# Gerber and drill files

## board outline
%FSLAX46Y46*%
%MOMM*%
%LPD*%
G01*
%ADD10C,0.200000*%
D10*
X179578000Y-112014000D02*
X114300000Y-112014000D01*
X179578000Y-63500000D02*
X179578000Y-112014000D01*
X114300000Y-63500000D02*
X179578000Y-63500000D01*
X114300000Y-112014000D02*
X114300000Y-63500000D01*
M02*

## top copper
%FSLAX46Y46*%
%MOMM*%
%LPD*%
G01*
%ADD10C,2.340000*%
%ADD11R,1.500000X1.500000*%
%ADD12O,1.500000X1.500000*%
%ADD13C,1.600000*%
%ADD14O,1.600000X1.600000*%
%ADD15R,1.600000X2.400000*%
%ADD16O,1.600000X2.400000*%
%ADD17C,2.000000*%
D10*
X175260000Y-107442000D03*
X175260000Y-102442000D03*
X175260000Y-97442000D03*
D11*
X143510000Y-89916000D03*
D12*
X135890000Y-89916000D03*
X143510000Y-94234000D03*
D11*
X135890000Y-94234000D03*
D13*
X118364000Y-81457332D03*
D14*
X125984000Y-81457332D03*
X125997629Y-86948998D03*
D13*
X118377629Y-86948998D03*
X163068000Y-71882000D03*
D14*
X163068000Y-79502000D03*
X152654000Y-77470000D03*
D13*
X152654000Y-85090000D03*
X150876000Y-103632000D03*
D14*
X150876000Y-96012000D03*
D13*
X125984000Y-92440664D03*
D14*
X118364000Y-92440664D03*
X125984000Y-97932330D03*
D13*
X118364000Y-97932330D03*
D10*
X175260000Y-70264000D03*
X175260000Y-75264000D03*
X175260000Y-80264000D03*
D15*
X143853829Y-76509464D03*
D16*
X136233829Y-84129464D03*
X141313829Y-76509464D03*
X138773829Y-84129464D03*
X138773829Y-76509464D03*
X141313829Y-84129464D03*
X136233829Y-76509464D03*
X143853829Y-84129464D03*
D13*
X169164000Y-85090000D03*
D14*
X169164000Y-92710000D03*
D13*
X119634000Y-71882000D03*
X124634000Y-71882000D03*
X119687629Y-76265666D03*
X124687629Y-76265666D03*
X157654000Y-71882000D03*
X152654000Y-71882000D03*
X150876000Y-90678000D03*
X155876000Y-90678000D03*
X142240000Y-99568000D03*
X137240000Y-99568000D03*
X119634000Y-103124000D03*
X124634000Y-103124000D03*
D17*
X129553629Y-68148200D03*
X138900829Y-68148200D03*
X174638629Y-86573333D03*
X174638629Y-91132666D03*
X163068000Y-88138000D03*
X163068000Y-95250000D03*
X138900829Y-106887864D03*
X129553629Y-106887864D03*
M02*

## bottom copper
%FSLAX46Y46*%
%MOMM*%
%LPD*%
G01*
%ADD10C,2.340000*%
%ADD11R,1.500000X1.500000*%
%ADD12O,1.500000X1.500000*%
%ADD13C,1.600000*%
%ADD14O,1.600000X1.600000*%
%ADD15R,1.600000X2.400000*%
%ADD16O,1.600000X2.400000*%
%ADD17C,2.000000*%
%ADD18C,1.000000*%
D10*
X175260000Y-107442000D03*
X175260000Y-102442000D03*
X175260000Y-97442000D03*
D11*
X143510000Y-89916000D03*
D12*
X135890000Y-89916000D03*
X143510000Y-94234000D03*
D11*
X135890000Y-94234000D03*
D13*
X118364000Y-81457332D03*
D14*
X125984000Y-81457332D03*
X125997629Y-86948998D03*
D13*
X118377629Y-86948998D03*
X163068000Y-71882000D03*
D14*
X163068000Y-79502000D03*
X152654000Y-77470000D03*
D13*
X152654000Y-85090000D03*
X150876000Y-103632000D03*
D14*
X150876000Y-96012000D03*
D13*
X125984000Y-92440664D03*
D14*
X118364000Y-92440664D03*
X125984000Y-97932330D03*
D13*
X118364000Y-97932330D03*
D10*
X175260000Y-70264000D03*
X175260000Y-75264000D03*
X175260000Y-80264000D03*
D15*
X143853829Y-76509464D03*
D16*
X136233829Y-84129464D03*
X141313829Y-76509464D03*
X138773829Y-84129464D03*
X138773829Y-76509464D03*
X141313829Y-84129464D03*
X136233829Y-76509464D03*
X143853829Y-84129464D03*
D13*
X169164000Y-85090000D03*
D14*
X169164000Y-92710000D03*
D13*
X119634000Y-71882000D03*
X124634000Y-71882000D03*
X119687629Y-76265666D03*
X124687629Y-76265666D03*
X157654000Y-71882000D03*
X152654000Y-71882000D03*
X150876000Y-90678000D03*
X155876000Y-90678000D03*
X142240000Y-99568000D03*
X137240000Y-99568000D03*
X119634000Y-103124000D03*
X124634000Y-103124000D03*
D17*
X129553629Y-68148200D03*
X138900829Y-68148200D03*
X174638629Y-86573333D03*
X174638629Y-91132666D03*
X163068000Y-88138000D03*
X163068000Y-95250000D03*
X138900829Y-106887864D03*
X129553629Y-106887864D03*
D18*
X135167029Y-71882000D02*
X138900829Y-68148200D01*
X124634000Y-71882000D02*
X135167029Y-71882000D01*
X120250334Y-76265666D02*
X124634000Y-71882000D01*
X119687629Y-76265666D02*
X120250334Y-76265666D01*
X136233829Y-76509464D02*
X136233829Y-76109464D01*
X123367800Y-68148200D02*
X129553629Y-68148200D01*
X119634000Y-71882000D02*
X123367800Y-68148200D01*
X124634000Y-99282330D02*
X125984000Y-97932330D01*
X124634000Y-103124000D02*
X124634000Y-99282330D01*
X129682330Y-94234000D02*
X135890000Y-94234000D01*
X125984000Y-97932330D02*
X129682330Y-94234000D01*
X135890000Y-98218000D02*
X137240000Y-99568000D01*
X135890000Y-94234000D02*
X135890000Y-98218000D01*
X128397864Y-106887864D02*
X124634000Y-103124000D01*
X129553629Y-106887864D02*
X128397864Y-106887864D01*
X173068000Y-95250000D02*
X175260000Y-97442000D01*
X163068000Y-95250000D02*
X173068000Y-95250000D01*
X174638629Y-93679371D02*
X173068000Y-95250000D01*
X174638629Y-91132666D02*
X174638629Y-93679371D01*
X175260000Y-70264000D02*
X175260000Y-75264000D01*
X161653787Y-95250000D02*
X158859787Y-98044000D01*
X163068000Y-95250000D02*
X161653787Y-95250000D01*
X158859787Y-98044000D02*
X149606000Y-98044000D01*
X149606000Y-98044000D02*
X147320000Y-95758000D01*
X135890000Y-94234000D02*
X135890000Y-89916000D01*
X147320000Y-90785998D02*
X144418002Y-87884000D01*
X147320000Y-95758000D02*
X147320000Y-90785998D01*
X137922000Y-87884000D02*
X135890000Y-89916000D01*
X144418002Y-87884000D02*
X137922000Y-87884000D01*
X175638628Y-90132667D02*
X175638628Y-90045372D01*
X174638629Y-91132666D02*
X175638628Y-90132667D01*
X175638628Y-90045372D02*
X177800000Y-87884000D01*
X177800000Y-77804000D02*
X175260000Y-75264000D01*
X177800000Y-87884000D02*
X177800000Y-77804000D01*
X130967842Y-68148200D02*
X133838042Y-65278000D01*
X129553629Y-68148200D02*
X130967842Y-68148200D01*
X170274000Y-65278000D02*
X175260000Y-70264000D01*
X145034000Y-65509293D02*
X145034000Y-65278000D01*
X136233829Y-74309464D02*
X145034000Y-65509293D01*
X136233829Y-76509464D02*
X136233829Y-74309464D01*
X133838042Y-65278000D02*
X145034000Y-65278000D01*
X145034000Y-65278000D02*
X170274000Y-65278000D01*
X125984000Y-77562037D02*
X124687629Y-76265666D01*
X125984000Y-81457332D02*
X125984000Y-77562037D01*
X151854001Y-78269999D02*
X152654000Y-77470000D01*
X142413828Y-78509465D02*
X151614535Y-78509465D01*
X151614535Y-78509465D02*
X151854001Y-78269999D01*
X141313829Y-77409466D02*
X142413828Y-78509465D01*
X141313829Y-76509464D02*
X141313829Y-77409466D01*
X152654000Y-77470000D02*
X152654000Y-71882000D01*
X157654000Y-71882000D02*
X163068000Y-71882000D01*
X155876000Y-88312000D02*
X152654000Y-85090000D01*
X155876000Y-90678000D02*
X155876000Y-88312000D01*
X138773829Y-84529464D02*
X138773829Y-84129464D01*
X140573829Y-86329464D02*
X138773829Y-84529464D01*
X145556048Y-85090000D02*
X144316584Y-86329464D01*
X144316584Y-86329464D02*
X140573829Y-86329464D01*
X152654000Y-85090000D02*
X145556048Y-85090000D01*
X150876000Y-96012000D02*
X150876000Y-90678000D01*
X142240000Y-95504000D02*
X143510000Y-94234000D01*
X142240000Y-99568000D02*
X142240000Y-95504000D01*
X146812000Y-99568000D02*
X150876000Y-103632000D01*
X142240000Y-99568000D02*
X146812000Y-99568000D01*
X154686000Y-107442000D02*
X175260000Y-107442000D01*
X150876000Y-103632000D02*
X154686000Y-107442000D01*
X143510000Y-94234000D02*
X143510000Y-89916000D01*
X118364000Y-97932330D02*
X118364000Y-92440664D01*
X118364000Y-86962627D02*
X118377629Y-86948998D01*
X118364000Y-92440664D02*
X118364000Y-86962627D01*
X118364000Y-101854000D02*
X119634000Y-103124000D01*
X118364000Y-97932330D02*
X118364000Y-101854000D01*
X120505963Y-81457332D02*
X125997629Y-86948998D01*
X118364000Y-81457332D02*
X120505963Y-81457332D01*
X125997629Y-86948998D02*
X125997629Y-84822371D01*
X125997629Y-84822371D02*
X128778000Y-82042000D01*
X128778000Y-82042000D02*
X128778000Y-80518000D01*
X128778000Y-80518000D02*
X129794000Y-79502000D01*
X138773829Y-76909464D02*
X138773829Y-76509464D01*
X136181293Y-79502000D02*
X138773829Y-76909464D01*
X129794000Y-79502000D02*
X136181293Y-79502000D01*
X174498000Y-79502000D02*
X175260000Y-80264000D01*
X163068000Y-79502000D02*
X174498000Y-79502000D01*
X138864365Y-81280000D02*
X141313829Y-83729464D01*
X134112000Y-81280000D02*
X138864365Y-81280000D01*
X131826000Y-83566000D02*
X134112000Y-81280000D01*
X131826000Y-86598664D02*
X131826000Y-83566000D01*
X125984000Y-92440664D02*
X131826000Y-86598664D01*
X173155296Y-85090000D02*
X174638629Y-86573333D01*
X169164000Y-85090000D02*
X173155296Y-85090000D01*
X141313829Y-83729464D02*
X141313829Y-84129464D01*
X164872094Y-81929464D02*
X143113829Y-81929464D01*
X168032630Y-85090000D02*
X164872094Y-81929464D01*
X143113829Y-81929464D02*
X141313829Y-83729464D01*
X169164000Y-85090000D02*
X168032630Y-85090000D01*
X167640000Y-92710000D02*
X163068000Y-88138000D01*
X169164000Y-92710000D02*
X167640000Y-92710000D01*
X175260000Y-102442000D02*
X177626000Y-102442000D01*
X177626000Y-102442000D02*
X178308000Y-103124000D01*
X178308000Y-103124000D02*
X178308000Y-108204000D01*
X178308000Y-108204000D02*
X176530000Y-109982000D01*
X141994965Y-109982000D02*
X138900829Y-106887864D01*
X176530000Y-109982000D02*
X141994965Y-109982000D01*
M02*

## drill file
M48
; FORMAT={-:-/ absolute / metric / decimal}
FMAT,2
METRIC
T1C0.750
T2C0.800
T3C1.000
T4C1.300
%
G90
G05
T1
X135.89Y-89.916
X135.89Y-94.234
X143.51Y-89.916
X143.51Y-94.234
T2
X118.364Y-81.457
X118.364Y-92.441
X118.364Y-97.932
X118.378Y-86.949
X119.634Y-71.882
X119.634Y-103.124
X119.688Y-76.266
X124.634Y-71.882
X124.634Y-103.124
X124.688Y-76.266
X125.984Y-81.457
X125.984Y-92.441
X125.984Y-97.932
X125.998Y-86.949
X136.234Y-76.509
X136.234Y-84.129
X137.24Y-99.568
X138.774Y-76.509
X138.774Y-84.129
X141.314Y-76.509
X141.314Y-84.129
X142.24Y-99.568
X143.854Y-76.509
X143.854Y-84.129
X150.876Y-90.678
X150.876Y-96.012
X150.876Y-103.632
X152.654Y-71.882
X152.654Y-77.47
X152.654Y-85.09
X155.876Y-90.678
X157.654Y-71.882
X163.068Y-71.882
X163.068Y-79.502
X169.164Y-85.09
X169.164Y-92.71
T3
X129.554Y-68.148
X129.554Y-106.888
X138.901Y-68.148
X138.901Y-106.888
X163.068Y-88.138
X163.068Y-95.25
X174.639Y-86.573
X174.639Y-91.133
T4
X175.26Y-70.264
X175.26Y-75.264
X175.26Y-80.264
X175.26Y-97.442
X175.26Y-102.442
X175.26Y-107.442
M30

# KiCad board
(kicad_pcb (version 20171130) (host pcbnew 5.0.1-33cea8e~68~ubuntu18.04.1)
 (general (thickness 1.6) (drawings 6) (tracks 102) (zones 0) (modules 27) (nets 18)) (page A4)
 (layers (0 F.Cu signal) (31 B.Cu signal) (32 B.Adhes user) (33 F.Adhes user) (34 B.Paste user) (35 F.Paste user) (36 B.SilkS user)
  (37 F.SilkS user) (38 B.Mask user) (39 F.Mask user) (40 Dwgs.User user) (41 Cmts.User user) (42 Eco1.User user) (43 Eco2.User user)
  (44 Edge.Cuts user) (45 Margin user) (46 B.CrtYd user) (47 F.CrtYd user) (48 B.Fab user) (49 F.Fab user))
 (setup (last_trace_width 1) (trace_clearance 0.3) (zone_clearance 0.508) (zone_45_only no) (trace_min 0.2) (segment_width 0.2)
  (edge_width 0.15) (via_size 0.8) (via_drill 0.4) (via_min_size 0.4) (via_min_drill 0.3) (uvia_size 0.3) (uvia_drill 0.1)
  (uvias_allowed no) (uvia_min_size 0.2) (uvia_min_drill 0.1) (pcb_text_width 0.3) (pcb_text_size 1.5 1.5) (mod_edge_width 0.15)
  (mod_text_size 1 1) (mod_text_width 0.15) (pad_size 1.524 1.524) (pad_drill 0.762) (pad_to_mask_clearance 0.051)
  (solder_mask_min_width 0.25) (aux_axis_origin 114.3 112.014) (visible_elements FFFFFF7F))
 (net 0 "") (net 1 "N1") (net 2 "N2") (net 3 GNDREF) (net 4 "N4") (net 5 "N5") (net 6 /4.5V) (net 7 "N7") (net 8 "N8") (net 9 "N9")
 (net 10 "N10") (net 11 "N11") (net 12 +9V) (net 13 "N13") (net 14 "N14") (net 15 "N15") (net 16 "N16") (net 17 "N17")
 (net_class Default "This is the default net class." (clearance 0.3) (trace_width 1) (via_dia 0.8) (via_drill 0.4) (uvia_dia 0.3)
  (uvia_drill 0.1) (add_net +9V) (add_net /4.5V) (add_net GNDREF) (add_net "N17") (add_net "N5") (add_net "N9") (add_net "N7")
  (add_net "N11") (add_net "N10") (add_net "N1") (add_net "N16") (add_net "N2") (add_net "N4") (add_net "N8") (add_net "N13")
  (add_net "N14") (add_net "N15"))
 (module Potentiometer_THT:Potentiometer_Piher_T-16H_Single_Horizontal (layer F.Cu) (at 175.26 107.442)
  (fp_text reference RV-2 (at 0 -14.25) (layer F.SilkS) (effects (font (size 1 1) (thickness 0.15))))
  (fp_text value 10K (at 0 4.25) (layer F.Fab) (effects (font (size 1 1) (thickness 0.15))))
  (pad 1 thru_hole circle (at 0 0) (size 2.34 2.34) (drill 1.3) (layers *.Cu *.Mask) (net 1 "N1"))
  (pad 2 thru_hole circle (at 0 -5) (size 2.34 2.34) (drill 1.3) (layers *.Cu *.Mask) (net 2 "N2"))
  (pad 3 thru_hole circle (at 0 -10) (size 2.34 2.34) (drill 1.3) (layers *.Cu *.Mask) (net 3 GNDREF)))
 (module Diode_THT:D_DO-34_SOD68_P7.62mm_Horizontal (layer F.Cu) (at 143.51 89.916 180)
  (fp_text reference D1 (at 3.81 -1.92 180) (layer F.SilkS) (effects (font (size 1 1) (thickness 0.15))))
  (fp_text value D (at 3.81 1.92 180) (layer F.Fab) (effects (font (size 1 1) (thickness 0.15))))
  (pad 1 thru_hole rect (at 0 0 180) (size 1.5 1.5) (drill 0.75) (layers *.Cu *.Mask) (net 1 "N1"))
  (pad 2 thru_hole oval (at 7.62 0 180) (size 1.5 1.5) (drill 0.75) (layers *.Cu *.Mask) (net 3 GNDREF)))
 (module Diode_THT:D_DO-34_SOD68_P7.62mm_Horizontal (layer F.Cu) (at 135.89 94.234)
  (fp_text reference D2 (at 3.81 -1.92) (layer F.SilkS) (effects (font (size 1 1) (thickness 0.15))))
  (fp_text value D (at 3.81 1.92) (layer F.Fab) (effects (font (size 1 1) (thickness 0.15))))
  (pad 2 thru_hole oval (at 7.62 0) (size 1.5 1.5) (drill 0.75) (layers *.Cu *.Mask) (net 1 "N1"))
  (pad 1 thru_hole rect (at 0 0) (size 1.5 1.5) (drill 0.75) (layers *.Cu *.Mask) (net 3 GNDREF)))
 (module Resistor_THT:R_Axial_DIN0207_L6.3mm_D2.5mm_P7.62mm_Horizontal (layer F.Cu) (at 118.364 81.457332)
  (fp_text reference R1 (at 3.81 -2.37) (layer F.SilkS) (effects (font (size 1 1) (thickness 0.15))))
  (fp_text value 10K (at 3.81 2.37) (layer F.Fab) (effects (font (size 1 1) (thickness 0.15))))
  (pad 1 thru_hole circle (at 0 0) (size 1.6 1.6) (drill 0.8) (layers *.Cu *.Mask) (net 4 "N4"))
  (pad 2 thru_hole oval (at 7.62 0) (size 1.6 1.6) (drill 0.8) (layers *.Cu *.Mask) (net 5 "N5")))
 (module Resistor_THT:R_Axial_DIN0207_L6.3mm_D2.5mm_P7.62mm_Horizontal (layer F.Cu) (at 118.377629 86.948998)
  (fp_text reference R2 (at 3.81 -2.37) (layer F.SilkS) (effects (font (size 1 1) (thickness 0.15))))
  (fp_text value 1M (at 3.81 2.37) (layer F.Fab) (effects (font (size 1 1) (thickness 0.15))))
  (pad 2 thru_hole oval (at 7.62 0) (size 1.6 1.6) (drill 0.8) (layers *.Cu *.Mask) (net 4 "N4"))
  (pad 1 thru_hole circle (at 0 0) (size 1.6 1.6) (drill 0.8) (layers *.Cu *.Mask) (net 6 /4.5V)))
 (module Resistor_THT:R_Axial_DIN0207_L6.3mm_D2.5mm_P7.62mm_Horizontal (layer F.Cu) (at 163.068 71.882 270)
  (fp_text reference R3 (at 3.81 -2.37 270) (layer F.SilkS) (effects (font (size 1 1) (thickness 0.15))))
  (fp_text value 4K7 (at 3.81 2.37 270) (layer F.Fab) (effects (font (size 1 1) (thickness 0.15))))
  (pad 1 thru_hole circle (at 0 0 270) (size 1.6 1.6) (drill 0.8) (layers *.Cu *.Mask) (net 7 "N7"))
  (pad 2 thru_hole oval (at 7.62 0 270) (size 1.6 1.6) (drill 0.8) (layers *.Cu *.Mask) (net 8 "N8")))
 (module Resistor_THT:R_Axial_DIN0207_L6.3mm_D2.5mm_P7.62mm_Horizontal (layer F.Cu) (at 152.654 85.09 90)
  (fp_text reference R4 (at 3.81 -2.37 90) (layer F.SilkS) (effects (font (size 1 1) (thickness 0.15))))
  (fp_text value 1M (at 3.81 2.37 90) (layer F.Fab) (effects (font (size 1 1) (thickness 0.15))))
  (pad 2 thru_hole oval (at 7.62 0 90) (size 1.6 1.6) (drill 0.8) (layers *.Cu *.Mask) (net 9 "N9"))
  (pad 1 thru_hole circle (at 0 0 90) (size 1.6 1.6) (drill 0.8) (layers *.Cu *.Mask) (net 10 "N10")))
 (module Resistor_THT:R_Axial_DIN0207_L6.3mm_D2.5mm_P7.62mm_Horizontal (layer F.Cu) (at 150.876 103.632 90)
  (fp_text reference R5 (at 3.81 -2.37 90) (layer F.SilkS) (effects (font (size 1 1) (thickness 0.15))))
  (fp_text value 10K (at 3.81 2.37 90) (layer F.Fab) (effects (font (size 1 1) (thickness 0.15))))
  (pad 1 thru_hole circle (at 0 0 90) (size 1.6 1.6) (drill 0.8) (layers *.Cu *.Mask) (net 1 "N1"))
  (pad 2 thru_hole oval (at 7.62 0 90) (size 1.6 1.6) (drill 0.8) (layers *.Cu *.Mask) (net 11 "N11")))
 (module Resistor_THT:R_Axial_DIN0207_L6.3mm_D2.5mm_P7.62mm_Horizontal (layer F.Cu) (at 125.984 92.440664 180)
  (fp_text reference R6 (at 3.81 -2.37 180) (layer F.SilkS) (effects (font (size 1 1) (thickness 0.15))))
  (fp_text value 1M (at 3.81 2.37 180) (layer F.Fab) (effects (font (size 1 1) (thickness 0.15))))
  (pad 1 thru_hole circle (at 0 0 180) (size 1.6 1.6) (drill 0.8) (layers *.Cu *.Mask) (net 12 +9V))
  (pad 2 thru_hole oval (at 7.62 0 180) (size 1.6 1.6) (drill 0.8) (layers *.Cu *.Mask) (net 6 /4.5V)))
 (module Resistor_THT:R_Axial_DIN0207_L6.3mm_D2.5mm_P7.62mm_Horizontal (layer F.Cu) (at 118.364 97.93233)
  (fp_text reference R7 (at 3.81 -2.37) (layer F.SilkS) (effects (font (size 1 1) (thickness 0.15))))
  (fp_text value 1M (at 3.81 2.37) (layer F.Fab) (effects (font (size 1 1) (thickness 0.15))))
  (pad 2 thru_hole oval (at 7.62 0) (size 1.6 1.6) (drill 0.8) (layers *.Cu *.Mask) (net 3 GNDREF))
  (pad 1 thru_hole circle (at 0 0) (size 1.6 1.6) (drill 0.8) (layers *.Cu *.Mask) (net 6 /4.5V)))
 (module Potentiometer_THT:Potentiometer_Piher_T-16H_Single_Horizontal (layer F.Cu) (at 175.26 80.264)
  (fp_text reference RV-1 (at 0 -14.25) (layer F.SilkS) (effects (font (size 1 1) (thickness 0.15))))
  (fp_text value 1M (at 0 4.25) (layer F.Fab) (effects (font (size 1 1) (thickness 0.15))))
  (pad 3 thru_hole circle (at 0 -10) (size 2.34 2.34) (drill 1.3) (layers *.Cu *.Mask) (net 3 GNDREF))
  (pad 2 thru_hole circle (at 0 -5) (size 2.34 2.34) (drill 1.3) (layers *.Cu *.Mask) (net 3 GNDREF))
  (pad 1 thru_hole circle (at 0 0) (size 2.34 2.34) (drill 1.3) (layers *.Cu *.Mask) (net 8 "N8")))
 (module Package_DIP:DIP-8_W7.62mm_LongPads (layer F.Cu) (at 143.853829 76.509464 270)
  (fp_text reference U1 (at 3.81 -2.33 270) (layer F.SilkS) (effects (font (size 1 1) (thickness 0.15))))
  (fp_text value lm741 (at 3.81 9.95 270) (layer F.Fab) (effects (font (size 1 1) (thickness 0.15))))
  (pad 1 thru_hole rect (at 0 0 270) (size 2.4 1.6) (drill 0.8) (layers *.Cu *.Mask) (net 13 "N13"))
  (pad 5 thru_hole oval (at 7.62 7.62 270) (size 2.4 1.6) (drill 0.8) (layers *.Cu *.Mask) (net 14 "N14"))
  (pad 2 thru_hole oval (at 0 2.54 270) (size 2.4 1.6) (drill 0.8) (layers *.Cu *.Mask) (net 9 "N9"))
  (pad 6 thru_hole oval (at 7.62 5.08 270) (size 2.4 1.6) (drill 0.8) (layers *.Cu *.Mask) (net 10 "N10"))
  (pad 3 thru_hole oval (at 0 5.08 270) (size 2.4 1.6) (drill 0.8) (layers *.Cu *.Mask) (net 4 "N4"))
  (pad 7 thru_hole oval (at 7.62 2.54 270) (size 2.4 1.6) (drill 0.8) (layers *.Cu *.Mask) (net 12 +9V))
  (pad 4 thru_hole oval (at 0 7.62 270) (size 2.4 1.6) (drill 0.8) (layers *.Cu *.Mask) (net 3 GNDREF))
  (pad 8 thru_hole oval (at 7.62 0 270) (size 2.4 1.6) (drill 0.8) (layers *.Cu *.Mask) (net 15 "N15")))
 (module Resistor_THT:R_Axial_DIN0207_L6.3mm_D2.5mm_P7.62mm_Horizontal (layer F.Cu) (at 169.164 85.09 270)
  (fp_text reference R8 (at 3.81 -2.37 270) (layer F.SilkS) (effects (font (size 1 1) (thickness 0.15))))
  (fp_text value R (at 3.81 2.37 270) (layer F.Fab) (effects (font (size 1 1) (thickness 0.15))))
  (pad 1 thru_hole circle (at 0 0 270) (size 1.6 1.6) (drill 0.8) (layers *.Cu *.Mask) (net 12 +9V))
  (pad 2 thru_hole oval (at 7.62 0 270) (size 1.6 1.6) (drill 0.8) (layers *.Cu *.Mask) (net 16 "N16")))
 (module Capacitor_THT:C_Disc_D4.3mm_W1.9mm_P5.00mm (layer F.Cu) (at 119.634 71.882)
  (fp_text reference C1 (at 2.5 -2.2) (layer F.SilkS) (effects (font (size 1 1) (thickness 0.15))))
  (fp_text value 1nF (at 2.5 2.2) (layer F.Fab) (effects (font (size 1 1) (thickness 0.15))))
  (pad 1 thru_hole circle (at 0 0) (size 1.6 1.6) (drill 0.8) (layers *.Cu *.Mask) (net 3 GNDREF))
  (pad 2 thru_hole circle (at 5 0) (size 1.6 1.6) (drill 0.8) (layers *.Cu *.Mask) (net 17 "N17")))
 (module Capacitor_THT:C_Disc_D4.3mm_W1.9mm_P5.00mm (layer F.Cu) (at 124.687629 76.265666 180)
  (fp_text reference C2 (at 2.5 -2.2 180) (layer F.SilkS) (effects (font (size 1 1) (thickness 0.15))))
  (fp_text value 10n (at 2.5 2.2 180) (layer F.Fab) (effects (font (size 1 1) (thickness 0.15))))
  (pad 2 thru_hole circle (at 5 0 180) (size 1.6 1.6) (drill 0.8) (layers *.Cu *.Mask) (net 17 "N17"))
  (pad 1 thru_hole circle (at 0 0 180) (size 1.6 1.6) (drill 0.8) (layers *.Cu *.Mask) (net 5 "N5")))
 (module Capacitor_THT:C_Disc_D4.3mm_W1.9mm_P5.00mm (layer F.Cu) (at 152.654 71.882)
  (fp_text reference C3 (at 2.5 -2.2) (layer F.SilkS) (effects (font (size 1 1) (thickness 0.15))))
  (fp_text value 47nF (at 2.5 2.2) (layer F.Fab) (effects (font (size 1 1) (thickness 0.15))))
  (pad 2 thru_hole circle (at 5 0) (size 1.6 1.6) (drill 0.8) (layers *.Cu *.Mask) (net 7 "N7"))
  (pad 1 thru_hole circle (at 0 0) (size 1.6 1.6) (drill 0.8) (layers *.Cu *.Mask) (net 9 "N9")))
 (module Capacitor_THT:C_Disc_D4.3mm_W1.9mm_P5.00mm (layer F.Cu) (at 150.876 90.678)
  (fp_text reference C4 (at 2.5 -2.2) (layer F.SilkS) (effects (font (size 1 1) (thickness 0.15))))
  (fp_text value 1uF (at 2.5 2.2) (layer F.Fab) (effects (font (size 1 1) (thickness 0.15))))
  (pad 1 thru_hole circle (at 0 0) (size 1.6 1.6) (drill 0.8) (layers *.Cu *.Mask) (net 11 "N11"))
  (pad 2 thru_hole circle (at 5 0) (size 1.6 1.6) (drill 0.8) (layers *.Cu *.Mask) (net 10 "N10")))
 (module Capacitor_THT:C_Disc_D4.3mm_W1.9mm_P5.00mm (layer F.Cu) (at 142.24 99.568 180)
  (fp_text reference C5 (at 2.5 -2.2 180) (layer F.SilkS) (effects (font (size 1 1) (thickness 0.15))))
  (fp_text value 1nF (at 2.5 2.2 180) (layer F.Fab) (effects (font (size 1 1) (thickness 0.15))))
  (pad 1 thru_hole circle (at 0 0 180) (size 1.6 1.6) (drill 0.8) (layers *.Cu *.Mask) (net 1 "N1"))
  (pad 2 thru_hole circle (at 5 0 180) (size 1.6 1.6) (drill 0.8) (layers *.Cu *.Mask) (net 3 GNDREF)))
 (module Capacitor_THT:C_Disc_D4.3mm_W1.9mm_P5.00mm (layer F.Cu) (at 119.634 103.124)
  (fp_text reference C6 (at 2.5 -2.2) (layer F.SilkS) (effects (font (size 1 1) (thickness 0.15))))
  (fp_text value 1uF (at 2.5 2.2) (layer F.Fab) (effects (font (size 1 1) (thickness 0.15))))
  (pad 1 thru_hole circle (at 0 0) (size 1.6 1.6) (drill 0.8) (layers *.Cu *.Mask) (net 6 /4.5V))
  (pad 2 thru_hole circle (at 5 0) (size 1.6 1.6) (drill 0.8) (layers *.Cu *.Mask) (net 3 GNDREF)))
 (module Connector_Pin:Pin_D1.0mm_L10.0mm (layer F.Cu) (at 129.553629 68.1482 180)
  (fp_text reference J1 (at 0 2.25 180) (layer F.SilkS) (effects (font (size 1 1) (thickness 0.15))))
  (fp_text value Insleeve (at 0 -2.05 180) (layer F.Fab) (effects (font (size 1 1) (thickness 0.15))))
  (pad 1 thru_hole circle (at 0 0 180) (size 2 2) (drill 1) (layers *.Cu *.Mask) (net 3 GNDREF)))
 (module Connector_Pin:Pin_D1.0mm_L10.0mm (layer F.Cu) (at 138.900829 68.1482 180)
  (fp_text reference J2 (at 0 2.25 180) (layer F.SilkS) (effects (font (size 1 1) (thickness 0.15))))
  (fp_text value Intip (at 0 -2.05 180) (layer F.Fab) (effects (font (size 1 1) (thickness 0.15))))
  (pad 1 thru_hole circle (at 0 0 180) (size 2 2) (drill 1) (layers *.Cu *.Mask) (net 17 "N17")))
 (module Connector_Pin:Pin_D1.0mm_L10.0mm (layer F.Cu) (at 174.638629 86.573333 270)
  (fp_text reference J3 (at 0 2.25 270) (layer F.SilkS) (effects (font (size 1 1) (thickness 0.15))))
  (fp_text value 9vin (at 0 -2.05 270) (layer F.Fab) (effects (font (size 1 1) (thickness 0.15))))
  (pad 1 thru_hole circle (at 0 0 270) (size 2 2) (drill 1) (layers *.Cu *.Mask) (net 12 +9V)))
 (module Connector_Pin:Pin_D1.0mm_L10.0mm (layer F.Cu) (at 174.638629 91.132666 270)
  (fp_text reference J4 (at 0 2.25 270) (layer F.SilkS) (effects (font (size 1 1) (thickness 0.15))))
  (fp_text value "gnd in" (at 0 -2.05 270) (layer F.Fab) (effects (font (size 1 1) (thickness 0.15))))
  (pad 1 thru_hole circle (at 0 0 270) (size 2 2) (drill 1) (layers *.Cu *.Mask) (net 3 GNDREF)))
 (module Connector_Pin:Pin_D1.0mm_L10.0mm (layer F.Cu) (at 163.068 88.138 270)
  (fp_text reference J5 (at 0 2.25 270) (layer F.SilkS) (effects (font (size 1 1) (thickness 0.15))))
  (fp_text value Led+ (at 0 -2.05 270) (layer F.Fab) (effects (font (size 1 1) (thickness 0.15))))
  (pad 1 thru_hole circle (at 0 0 270) (size 2 2) (drill 1) (layers *.Cu *.Mask) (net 16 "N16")))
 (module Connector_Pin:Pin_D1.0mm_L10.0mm (layer F.Cu) (at 163.068 95.25 270)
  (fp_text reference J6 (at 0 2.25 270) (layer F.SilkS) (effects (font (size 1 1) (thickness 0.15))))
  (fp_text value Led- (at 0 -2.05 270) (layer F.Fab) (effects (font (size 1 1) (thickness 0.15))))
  (pad 1 thru_hole circle (at 0 0 270) (size 2 2) (drill 1) (layers *.Cu *.Mask) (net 3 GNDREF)))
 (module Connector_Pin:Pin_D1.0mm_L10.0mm (layer F.Cu) (at 138.900829 106.887864)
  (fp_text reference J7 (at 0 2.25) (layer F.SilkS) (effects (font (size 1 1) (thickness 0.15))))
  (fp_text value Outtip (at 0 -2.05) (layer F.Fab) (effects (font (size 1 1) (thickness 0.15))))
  (pad 1 thru_hole circle (at 0 0) (size 2 2) (drill 1) (layers *.Cu *.Mask) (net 2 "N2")))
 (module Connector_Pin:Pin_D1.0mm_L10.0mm (layer F.Cu) (at 129.553629 106.887864)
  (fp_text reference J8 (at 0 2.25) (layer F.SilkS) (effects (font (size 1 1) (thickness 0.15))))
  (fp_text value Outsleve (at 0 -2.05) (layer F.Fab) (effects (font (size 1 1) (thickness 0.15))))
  (pad 1 thru_hole circle (at 0 0) (size 2 2) (drill 1) (layers *.Cu *.Mask) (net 3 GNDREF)))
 (gr_line (start 179.578 112.014) (end 114.3 112.014) (layer Edge.Cuts) (width 0.2))
 (gr_line (start 179.578 63.5) (end 179.578 112.014) (layer Edge.Cuts) (width 0.2))
 (gr_line (start 114.3 63.5) (end 179.578 63.5) (layer Edge.Cuts) (width 0.2))
 (gr_line (start 114.3 112.014) (end 114.3 63.5) (layer Edge.Cuts) (width 0.2))
 (segment (start 135.167029 71.882) (end 138.900829 68.1482) (width 1) (layer B.Cu) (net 17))
 (segment (start 124.634 71.882) (end 135.167029 71.882) (width 1) (layer B.Cu) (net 17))
 (segment (start 120.250334 76.265666) (end 124.634 71.882) (width 1) (layer B.Cu) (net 17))
 (segment (start 119.687629 76.265666) (end 120.250334 76.265666) (width 1) (layer B.Cu) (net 17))
 (segment (start 136.233829 76.509464) (end 136.233829 76.109464) (width 1) (layer B.Cu) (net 3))
 (segment (start 123.3678 68.1482) (end 129.553629 68.1482) (width 1) (layer B.Cu) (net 3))
 (segment (start 119.634 71.882) (end 123.3678 68.1482) (width 1) (layer B.Cu) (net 3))
 (segment (start 124.634 99.28233) (end 125.984 97.93233) (width 1) (layer B.Cu) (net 3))
 (segment (start 124.634 103.124) (end 124.634 99.28233) (width 1) (layer B.Cu) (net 3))
 (segment (start 129.68233 94.234) (end 135.89 94.234) (width 1) (layer B.Cu) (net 3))
 (segment (start 125.984 97.93233) (end 129.68233 94.234) (width 1) (layer B.Cu) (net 3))
 (segment (start 135.89 98.218) (end 137.24 99.568) (width 1) (layer B.Cu) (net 3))
 (segment (start 135.89 94.234) (end 135.89 98.218) (width 1) (layer B.Cu) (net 3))
 (segment (start 128.397864 106.887864) (end 124.634 103.124) (width 1) (layer B.Cu) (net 3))
 (segment (start 129.553629 106.887864) (end 128.397864 106.887864) (width 1) (layer B.Cu) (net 3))
 (segment (start 173.068 95.25) (end 175.26 97.442) (width 1) (layer B.Cu) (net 3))
 (segment (start 163.068 95.25) (end 173.068 95.25) (width 1) (layer B.Cu) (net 3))
 (segment (start 174.638629 93.679371) (end 173.068 95.25) (width 1) (layer B.Cu) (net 3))
 (segment (start 174.638629 91.132666) (end 174.638629 93.679371) (width 1) (layer B.Cu) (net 3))
 (segment (start 175.26 70.264) (end 175.26 75.264) (width 1) (layer B.Cu) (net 3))
 (segment (start 161.653787 95.25) (end 158.859787 98.044) (width 1) (layer B.Cu) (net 3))
 (segment (start 163.068 95.25) (end 161.653787 95.25) (width 1) (layer B.Cu) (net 3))
 (segment (start 158.859787 98.044) (end 149.606 98.044) (width 1) (layer B.Cu) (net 3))
 (segment (start 149.606 98.044) (end 147.32 95.758) (width 1) (layer B.Cu) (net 3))
 (segment (start 135.89 94.234) (end 135.89 89.916) (width 1) (layer B.Cu) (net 3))
 (segment (start 147.32 90.785998) (end 144.418002 87.884) (width 1) (layer B.Cu) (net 3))
 (segment (start 147.32 95.758) (end 147.32 90.785998) (width 1) (layer B.Cu) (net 3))
 (segment (start 137.922 87.884) (end 135.89 89.916) (width 1) (layer B.Cu) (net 3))
 (segment (start 144.418002 87.884) (end 137.922 87.884) (width 1) (layer B.Cu) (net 3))
 (segment (start 175.638628 90.132667) (end 175.638628 90.045372) (width 1) (layer B.Cu) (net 3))
 (segment (start 174.638629 91.132666) (end 175.638628 90.132667) (width 1) (layer B.Cu) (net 3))
 (segment (start 175.638628 90.045372) (end 177.8 87.884) (width 1) (layer B.Cu) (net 3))
 (segment (start 177.8 77.804) (end 175.26 75.264) (width 1) (layer B.Cu) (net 3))
 (segment (start 177.8 87.884) (end 177.8 77.804) (width 1) (layer B.Cu) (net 3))
 (segment (start 130.967842 68.1482) (end 133.838042 65.278) (width 1) (layer B.Cu) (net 3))
 (segment (start 129.553629 68.1482) (end 130.967842 68.1482) (width 1) (layer B.Cu) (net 3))
 (segment (start 170.274 65.278) (end 175.26 70.264) (width 1) (layer B.Cu) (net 3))
 (segment (start 145.034 65.509293) (end 145.034 65.278) (width 1) (layer B.Cu) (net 3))
 (segment (start 136.233829 74.309464) (end 145.034 65.509293) (width 1) (layer B.Cu) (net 3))
 (segment (start 136.233829 76.509464) (end 136.233829 74.309464) (width 1) (layer B.Cu) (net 3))
 (segment (start 133.838042 65.278) (end 145.034 65.278) (width 1) (layer B.Cu) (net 3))
 (segment (start 145.034 65.278) (end 170.274 65.278) (width 1) (layer B.Cu) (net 3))
 (segment (start 125.984 77.562037) (end 124.687629 76.265666) (width 1) (layer B.Cu) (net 5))
 (segment (start 125.984 81.457332) (end 125.984 77.562037) (width 1) (layer B.Cu) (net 5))
 (segment (start 151.854001 78.269999) (end 152.654 77.47) (width 1) (layer B.Cu) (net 9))
 (segment (start 142.413828 78.509465) (end 151.614535 78.509465) (width 1) (layer B.Cu) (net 9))
 (segment (start 151.614535 78.509465) (end 151.854001 78.269999) (width 1) (layer B.Cu) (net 9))
 (segment (start 141.313829 77.409466) (end 142.413828 78.509465) (width 1) (layer B.Cu) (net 9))
 (segment (start 141.313829 76.509464) (end 141.313829 77.409466) (width 1) (layer B.Cu) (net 9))
 (segment (start 152.654 77.47) (end 152.654 71.882) (width 1) (layer B.Cu) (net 9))
 (segment (start 157.654 71.882) (end 163.068 71.882) (width 1) (layer B.Cu) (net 7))
 (segment (start 155.876 88.312) (end 152.654 85.09) (width 1) (layer B.Cu) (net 10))
 (segment (start 155.876 90.678) (end 155.876 88.312) (width 1) (layer B.Cu) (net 10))
 (segment (start 138.773829 84.529464) (end 138.773829 84.129464) (width 1) (layer B.Cu) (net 10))
 (segment (start 140.573829 86.329464) (end 138.773829 84.529464) (width 1) (layer B.Cu) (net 10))
 (segment (start 145.556048 85.09) (end 144.316584 86.329464) (width 1) (layer B.Cu) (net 10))
 (segment (start 144.316584 86.329464) (end 140.573829 86.329464) (width 1) (layer B.Cu) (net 10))
 (segment (start 152.654 85.09) (end 145.556048 85.09) (width 1) (layer B.Cu) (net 10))
 (segment (start 150.876 96.012) (end 150.876 90.678) (width 1) (layer B.Cu) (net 11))
 (segment (start 142.24 95.504) (end 143.51 94.234) (width 1) (layer B.Cu) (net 1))
 (segment (start 142.24 99.568) (end 142.24 95.504) (width 1) (layer B.Cu) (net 1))
 (segment (start 146.812 99.568) (end 150.876 103.632) (width 1) (layer B.Cu) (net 1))
 (segment (start 142.24 99.568) (end 146.812 99.568) (width 1) (layer B.Cu) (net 1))
 (segment (start 154.686 107.442) (end 175.26 107.442) (width 1) (layer B.Cu) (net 1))
 (segment (start 150.876 103.632) (end 154.686 107.442) (width 1) (layer B.Cu) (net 1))
 (segment (start 143.51 94.234) (end 143.51 89.916) (width 1) (layer B.Cu) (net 1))
 (segment (start 118.364 97.93233) (end 118.364 92.440664) (width 1) (layer B.Cu) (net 6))
 (segment (start 118.364 86.962627) (end 118.377629 86.948998) (width 1) (layer B.Cu) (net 6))
 (segment (start 118.364 92.440664) (end 118.364 86.962627) (width 1) (layer B.Cu) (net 6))
 (segment (start 118.364 101.854) (end 119.634 103.124) (width 1) (layer B.Cu) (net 6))
 (segment (start 118.364 97.93233) (end 118.364 101.854) (width 1) (layer B.Cu) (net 6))
 (segment (start 120.505963 81.457332) (end 125.997629 86.948998) (width 1) (layer B.Cu) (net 4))
 (segment (start 118.364 81.457332) (end 120.505963 81.457332) (width 1) (layer B.Cu) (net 4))
 (segment (start 125.997629 86.948998) (end 125.997629 84.822371) (width 1) (layer B.Cu) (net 4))
 (segment (start 125.997629 84.822371) (end 128.778 82.042) (width 1) (layer B.Cu) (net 4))
 (segment (start 128.778 82.042) (end 128.778 80.518) (width 1) (layer B.Cu) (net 4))
 (segment (start 128.778 80.518) (end 129.794 79.502) (width 1) (layer B.Cu) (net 4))
 (segment (start 138.773829 76.909464) (end 138.773829 76.509464) (width 1) (layer B.Cu) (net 4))
 (segment (start 136.181293 79.502) (end 138.773829 76.909464) (width 1) (layer B.Cu) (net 4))
 (segment (start 129.794 79.502) (end 136.181293 79.502) (width 1) (layer B.Cu) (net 4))
 (segment (start 174.498 79.502) (end 175.26 80.264) (width 1) (layer B.Cu) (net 8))
 (segment (start 163.068 79.502) (end 174.498 79.502) (width 1) (layer B.Cu) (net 8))
 (segment (start 138.864365 81.28) (end 141.313829 83.729464) (width 1) (layer B.Cu) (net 12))
 (segment (start 134.112 81.28) (end 138.864365 81.28) (width 1) (layer B.Cu) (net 12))
 (segment (start 131.826 83.566) (end 134.112 81.28) (width 1) (layer B.Cu) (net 12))
 (segment (start 131.826 86.598664) (end 131.826 83.566) (width 1) (layer B.Cu) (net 12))
 (segment (start 125.984 92.440664) (end 131.826 86.598664) (width 1) (layer B.Cu) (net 12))
 (segment (start 173.155296 85.09) (end 174.638629 86.573333) (width 1) (layer B.Cu) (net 12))
 (segment (start 169.164 85.09) (end 173.155296 85.09) (width 1) (layer B.Cu) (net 12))
 (segment (start 141.313829 83.729464) (end 141.313829 84.129464) (width 1) (layer B.Cu) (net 12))
 (segment (start 164.872094 81.929464) (end 143.113829 81.929464) (width 1) (layer B.Cu) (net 12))
 (segment (start 168.03263 85.09) (end 164.872094 81.929464) (width 1) (layer B.Cu) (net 12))
 (segment (start 143.113829 81.929464) (end 141.313829 83.729464) (width 1) (layer B.Cu) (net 12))
 (segment (start 169.164 85.09) (end 168.03263 85.09) (width 1) (layer B.Cu) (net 12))
 (segment (start 167.64 92.71) (end 163.068 88.138) (width 1) (layer B.Cu) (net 16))
 (segment (start 169.164 92.71) (end 167.64 92.71) (width 1) (layer B.Cu) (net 16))
 (segment (start 175.26 102.442) (end 177.626 102.442) (width 1) (layer B.Cu) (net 2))
 (segment (start 177.626 102.442) (end 178.308 103.124) (width 1) (layer B.Cu) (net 2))
 (segment (start 178.308 103.124) (end 178.308 108.204) (width 1) (layer B.Cu) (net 2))
 (segment (start 178.308 108.204) (end 176.53 109.982) (width 1) (layer B.Cu) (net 2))
 (segment (start 141.994965 109.982) (end 138.900829 106.887864) (width 1) (layer B.Cu) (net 2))
 (segment (start 176.53 109.982) (end 141.994965 109.982) (width 1) (layer B.Cu) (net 2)))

